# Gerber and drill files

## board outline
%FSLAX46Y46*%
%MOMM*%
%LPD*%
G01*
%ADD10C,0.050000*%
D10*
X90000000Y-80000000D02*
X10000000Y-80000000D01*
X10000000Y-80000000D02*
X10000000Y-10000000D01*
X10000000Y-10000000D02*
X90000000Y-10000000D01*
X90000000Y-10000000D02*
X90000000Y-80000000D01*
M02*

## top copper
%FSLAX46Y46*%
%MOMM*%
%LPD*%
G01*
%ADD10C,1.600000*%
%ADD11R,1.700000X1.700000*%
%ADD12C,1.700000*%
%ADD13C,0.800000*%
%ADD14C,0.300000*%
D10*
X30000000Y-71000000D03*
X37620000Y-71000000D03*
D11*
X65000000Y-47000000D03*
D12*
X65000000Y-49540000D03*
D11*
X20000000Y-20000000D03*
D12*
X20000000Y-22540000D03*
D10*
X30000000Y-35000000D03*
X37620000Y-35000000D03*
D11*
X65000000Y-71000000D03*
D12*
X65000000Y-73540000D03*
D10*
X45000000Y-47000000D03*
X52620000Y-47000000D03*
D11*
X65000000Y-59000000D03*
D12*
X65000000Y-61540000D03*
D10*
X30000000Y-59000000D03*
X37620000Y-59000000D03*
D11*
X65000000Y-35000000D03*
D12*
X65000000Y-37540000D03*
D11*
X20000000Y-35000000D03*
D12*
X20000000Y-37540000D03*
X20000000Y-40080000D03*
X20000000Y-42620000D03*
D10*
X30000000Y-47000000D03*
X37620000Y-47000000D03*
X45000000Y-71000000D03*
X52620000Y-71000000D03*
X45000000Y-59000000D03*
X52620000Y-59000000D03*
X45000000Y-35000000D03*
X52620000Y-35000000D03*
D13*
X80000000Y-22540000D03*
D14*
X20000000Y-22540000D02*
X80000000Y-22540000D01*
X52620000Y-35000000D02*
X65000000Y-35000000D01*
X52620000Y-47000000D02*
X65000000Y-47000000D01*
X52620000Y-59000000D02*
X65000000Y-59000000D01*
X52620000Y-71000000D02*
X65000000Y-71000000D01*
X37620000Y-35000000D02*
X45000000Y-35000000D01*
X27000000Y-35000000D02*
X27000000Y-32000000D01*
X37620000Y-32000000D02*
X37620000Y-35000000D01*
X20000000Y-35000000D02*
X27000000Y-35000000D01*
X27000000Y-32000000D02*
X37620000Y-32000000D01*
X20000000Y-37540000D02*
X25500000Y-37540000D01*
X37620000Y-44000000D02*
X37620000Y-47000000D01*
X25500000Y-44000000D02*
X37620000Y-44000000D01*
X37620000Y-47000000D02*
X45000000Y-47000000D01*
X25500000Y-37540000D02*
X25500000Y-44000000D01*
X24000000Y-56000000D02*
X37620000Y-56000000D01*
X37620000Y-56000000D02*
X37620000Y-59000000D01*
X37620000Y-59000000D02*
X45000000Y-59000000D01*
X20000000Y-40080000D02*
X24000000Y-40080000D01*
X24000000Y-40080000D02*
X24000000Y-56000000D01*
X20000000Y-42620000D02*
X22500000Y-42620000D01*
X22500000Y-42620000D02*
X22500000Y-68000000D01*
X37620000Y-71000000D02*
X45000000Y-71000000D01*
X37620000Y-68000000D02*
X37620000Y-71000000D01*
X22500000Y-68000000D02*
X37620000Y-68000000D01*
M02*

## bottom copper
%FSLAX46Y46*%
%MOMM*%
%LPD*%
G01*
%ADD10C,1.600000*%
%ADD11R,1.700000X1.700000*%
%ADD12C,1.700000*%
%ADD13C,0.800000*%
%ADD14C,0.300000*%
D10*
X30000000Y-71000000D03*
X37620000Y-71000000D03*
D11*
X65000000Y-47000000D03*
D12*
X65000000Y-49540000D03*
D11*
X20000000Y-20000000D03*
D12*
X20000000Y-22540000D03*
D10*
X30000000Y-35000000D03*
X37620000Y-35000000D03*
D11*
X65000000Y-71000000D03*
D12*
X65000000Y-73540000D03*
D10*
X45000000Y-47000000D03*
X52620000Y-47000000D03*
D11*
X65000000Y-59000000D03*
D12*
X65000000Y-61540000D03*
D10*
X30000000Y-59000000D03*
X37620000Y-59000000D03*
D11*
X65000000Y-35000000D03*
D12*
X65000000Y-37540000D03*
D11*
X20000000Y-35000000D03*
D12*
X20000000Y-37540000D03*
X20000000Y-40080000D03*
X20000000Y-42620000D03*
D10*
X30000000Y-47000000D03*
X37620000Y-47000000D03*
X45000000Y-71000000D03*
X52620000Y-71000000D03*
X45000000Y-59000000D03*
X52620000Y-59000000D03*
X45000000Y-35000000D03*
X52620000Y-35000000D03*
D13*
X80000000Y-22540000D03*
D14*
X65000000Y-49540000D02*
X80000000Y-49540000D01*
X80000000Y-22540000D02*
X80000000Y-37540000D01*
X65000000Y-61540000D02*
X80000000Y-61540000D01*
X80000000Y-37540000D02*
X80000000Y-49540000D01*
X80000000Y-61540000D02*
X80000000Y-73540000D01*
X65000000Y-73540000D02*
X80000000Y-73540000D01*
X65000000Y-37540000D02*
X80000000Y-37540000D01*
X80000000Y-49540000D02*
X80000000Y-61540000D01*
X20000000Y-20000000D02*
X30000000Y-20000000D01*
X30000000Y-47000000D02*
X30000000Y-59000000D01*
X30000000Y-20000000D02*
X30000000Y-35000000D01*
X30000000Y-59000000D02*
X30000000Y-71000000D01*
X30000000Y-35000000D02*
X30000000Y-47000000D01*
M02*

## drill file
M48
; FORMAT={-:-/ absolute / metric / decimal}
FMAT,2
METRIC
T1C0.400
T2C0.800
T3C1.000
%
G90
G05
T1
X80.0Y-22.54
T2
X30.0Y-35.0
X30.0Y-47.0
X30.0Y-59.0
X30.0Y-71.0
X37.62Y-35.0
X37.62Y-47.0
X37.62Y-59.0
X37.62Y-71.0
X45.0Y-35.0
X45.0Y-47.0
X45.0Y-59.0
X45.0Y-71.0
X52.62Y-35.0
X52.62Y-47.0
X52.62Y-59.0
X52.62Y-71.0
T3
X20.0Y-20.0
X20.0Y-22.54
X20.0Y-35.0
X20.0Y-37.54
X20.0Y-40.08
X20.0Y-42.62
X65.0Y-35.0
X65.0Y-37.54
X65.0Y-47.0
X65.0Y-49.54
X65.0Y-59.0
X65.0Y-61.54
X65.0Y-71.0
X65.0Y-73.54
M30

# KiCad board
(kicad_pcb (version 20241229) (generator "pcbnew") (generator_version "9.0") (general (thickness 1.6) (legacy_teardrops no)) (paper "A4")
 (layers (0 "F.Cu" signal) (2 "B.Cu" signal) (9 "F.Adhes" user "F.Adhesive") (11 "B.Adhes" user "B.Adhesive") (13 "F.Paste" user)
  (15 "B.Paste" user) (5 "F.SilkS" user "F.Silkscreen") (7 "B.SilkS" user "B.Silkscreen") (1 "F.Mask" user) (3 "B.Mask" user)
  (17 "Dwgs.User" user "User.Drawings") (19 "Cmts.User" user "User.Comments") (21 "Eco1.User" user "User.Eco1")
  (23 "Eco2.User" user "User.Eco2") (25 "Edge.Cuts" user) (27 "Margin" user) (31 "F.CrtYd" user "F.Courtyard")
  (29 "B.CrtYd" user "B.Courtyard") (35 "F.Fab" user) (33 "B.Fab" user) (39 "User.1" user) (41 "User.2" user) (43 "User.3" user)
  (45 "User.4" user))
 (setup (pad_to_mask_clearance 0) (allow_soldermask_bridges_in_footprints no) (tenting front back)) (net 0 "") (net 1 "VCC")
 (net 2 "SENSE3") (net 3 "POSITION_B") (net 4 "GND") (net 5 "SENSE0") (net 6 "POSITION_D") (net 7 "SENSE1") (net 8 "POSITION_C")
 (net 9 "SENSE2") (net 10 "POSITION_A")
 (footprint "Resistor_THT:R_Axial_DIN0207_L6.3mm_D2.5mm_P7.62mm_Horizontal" (layer "F.Cu") (at 30 71)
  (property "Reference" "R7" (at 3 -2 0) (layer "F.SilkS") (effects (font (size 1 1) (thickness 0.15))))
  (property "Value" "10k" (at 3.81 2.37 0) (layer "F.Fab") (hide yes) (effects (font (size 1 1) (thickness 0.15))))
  (pad "1" thru_hole circle (at 0 0) (size 1.6 1.6) (drill 0.8) (layers "*.Cu" "*.Mask") (remove_unused_layers no) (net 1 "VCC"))
  (pad "2" thru_hole circle (at 7.62 0) (size 1.6 1.6) (drill 0.8) (layers "*.Cu" "*.Mask") (remove_unused_layers no) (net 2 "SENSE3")))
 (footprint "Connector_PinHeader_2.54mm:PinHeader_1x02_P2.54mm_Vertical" (layer "F.Cu") (at 65 47)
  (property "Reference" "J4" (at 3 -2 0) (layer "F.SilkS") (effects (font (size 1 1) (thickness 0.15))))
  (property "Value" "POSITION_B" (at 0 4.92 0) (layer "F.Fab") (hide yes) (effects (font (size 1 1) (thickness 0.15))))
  (pad "1" thru_hole rect (at 0 0) (size 1.7 1.7) (drill 1) (layers "*.Cu" "*.Mask") (remove_unused_layers no) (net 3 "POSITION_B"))
  (pad "2" thru_hole circle (at 0 2.54) (size 1.7 1.7) (drill 1) (layers "*.Cu" "*.Mask") (remove_unused_layers no) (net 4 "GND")))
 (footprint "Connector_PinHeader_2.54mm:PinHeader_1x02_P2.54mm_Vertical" (layer "F.Cu") (at 20 20)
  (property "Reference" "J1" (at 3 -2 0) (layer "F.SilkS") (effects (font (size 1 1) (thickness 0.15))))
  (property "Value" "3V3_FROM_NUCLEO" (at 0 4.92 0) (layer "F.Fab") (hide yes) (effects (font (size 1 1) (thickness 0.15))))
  (pad "1" thru_hole rect (at 0 0) (size 1.7 1.7) (drill 1) (layers "*.Cu" "*.Mask") (remove_unused_layers no) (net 1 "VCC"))
  (pad "2" thru_hole circle (at 0 2.54) (size 1.7 1.7) (drill 1) (layers "*.Cu" "*.Mask") (remove_unused_layers no) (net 4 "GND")))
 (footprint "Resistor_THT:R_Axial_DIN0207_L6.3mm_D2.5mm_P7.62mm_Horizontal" (layer "F.Cu") (at 30 35)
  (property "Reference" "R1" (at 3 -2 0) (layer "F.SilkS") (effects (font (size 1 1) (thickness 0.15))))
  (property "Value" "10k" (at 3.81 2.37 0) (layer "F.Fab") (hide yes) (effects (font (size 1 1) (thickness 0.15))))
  (pad "1" thru_hole circle (at 0 0) (size 1.6 1.6) (drill 0.8) (layers "*.Cu" "*.Mask") (remove_unused_layers no) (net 1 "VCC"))
  (pad "2" thru_hole circle (at 7.62 0) (size 1.6 1.6) (drill 0.8) (layers "*.Cu" "*.Mask") (remove_unused_layers no) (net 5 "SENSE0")))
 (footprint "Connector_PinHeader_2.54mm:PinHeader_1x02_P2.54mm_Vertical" (layer "F.Cu") (at 65 71)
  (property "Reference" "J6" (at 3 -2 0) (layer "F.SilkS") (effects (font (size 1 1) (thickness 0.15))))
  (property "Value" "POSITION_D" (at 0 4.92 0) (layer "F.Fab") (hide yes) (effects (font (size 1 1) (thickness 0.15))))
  (pad "1" thru_hole rect (at 0 0) (size 1.7 1.7) (drill 1) (layers "*.Cu" "*.Mask") (remove_unused_layers no) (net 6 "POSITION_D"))
  (pad "2" thru_hole circle (at 0 2.54) (size 1.7 1.7) (drill 1) (layers "*.Cu" "*.Mask") (remove_unused_layers no) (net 4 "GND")))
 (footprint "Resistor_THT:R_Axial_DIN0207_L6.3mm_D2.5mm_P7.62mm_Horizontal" (layer "F.Cu") (at 45 47)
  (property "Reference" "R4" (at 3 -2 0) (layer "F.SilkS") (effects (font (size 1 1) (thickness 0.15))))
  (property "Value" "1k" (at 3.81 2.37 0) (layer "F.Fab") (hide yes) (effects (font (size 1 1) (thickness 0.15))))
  (pad "1" thru_hole circle (at 0 0) (size 1.6 1.6) (drill 0.8) (layers "*.Cu" "*.Mask") (remove_unused_layers no) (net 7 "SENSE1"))
  (pad "2" thru_hole circle (at 7.62 0) (size 1.6 1.6) (drill 0.8) (layers "*.Cu" "*.Mask") (remove_unused_layers no) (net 3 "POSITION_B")))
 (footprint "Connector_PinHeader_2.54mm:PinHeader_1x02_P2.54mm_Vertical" (layer "F.Cu") (at 65 59)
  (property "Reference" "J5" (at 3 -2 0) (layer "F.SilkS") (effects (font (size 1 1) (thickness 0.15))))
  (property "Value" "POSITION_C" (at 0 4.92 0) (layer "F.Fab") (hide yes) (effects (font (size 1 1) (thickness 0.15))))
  (pad "1" thru_hole rect (at 0 0) (size 1.7 1.7) (drill 1) (layers "*.Cu" "*.Mask") (remove_unused_layers no) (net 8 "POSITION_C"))
  (pad "2" thru_hole circle (at 0 2.54) (size 1.7 1.7) (drill 1) (layers "*.Cu" "*.Mask") (remove_unused_layers no) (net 4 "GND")))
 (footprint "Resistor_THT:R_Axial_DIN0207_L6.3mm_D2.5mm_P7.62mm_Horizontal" (layer "F.Cu") (at 30 59)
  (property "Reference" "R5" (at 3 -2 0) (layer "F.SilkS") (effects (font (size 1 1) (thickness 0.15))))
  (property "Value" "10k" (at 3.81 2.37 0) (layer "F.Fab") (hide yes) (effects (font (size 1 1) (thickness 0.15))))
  (pad "1" thru_hole circle (at 0 0) (size 1.6 1.6) (drill 0.8) (layers "*.Cu" "*.Mask") (remove_unused_layers no) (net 1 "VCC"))
  (pad "2" thru_hole circle (at 7.62 0) (size 1.6 1.6) (drill 0.8) (layers "*.Cu" "*.Mask") (remove_unused_layers no) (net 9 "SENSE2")))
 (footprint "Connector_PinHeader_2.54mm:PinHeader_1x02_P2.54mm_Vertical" (layer "F.Cu") (at 65 35)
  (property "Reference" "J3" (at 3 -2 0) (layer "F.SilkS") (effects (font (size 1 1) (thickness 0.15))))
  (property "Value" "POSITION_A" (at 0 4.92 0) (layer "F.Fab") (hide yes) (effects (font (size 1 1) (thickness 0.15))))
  (pad "1" thru_hole rect (at 0 0) (size 1.7 1.7) (drill 1) (layers "*.Cu" "*.Mask") (remove_unused_layers no) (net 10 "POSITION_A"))
  (pad "2" thru_hole circle (at 0 2.54) (size 1.7 1.7) (drill 1) (layers "*.Cu" "*.Mask") (remove_unused_layers no) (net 4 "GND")))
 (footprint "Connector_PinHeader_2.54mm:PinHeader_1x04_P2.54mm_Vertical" (layer "F.Cu") (at 20 35)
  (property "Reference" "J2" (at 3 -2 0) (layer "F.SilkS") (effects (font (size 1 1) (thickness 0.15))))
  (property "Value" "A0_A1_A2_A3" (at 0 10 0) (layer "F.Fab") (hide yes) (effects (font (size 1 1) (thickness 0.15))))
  (pad "1" thru_hole rect (at 0 0) (size 1.7 1.7) (drill 1) (layers "*.Cu" "*.Mask") (remove_unused_layers no) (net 5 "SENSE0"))
  (pad "2" thru_hole circle (at 0 2.54) (size 1.7 1.7) (drill 1) (layers "*.Cu" "*.Mask") (remove_unused_layers no) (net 7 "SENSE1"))
  (pad "3" thru_hole circle (at 0 5.08) (size 1.7 1.7) (drill 1) (layers "*.Cu" "*.Mask") (remove_unused_layers no) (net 9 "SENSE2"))
  (pad "4" thru_hole circle (at 0 7.62) (size 1.7 1.7) (drill 1) (layers "*.Cu" "*.Mask") (remove_unused_layers no) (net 2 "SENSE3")))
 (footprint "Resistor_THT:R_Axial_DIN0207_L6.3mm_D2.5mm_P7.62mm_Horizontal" (layer "F.Cu") (at 30 47)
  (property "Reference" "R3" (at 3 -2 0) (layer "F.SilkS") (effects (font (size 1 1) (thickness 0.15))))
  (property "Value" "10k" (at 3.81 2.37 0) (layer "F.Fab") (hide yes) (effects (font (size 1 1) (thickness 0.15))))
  (pad "1" thru_hole circle (at 0 0) (size 1.6 1.6) (drill 0.8) (layers "*.Cu" "*.Mask") (remove_unused_layers no) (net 1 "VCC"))
  (pad "2" thru_hole circle (at 7.62 0) (size 1.6 1.6) (drill 0.8) (layers "*.Cu" "*.Mask") (remove_unused_layers no) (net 7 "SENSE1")))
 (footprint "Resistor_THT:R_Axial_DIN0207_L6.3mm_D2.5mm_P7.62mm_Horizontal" (layer "F.Cu") (at 45 71)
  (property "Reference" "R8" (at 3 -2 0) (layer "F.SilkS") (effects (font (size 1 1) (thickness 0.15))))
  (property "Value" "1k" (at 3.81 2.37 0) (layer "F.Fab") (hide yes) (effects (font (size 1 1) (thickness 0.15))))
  (pad "1" thru_hole circle (at 0 0) (size 1.6 1.6) (drill 0.8) (layers "*.Cu" "*.Mask") (remove_unused_layers no) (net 2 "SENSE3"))
  (pad "2" thru_hole circle (at 7.62 0) (size 1.6 1.6) (drill 0.8) (layers "*.Cu" "*.Mask") (remove_unused_layers no) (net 6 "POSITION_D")))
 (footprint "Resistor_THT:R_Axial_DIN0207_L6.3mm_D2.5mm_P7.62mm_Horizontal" (layer "F.Cu") (at 45 59)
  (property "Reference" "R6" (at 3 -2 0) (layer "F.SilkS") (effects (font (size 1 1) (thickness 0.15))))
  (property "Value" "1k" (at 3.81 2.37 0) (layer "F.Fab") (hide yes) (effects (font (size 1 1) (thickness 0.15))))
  (pad "1" thru_hole circle (at 0 0) (size 1.6 1.6) (drill 0.8) (layers "*.Cu" "*.Mask") (remove_unused_layers no) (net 9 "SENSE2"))
  (pad "2" thru_hole circle (at 7.62 0) (size 1.6 1.6) (drill 0.8) (layers "*.Cu" "*.Mask") (remove_unused_layers no) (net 8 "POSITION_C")))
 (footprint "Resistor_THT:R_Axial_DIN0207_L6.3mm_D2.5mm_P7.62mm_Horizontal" (layer "F.Cu") (at 45 35)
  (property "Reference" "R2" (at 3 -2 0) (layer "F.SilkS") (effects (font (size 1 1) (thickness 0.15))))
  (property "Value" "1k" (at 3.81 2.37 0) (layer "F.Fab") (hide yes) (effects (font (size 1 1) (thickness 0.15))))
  (pad "1" thru_hole circle (at 0 0) (size 1.6 1.6) (drill 0.8) (layers "*.Cu" "*.Mask") (remove_unused_layers no) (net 5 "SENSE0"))
  (pad "2" thru_hole circle (at 7.62 0) (size 1.6 1.6) (drill 0.8) (layers "*.Cu" "*.Mask") (remove_unused_layers no) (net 10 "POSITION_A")))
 (gr_line (start 90 80) (end 10 80) (stroke (width 0.05) (type default)) (layer "Edge.Cuts"))
 (gr_line (start 10 80) (end 10 10) (stroke (width 0.05) (type default)) (layer "Edge.Cuts"))
 (gr_line (start 10 10) (end 90 10) (stroke (width 0.05) (type default)) (layer "Edge.Cuts"))
 (gr_line (start 90 10) (end 90 80) (stroke (width 0.05) (type default)) (layer "Edge.Cuts"))
 (segment (start 20 22.54) (end 80 22.54) (width 0.3) (layer "F.Cu") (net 4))
 (via (at 80 22.54) (size 0.8) (drill 0.4) (layers "F.Cu" "B.Cu") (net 4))
 (segment (start 65 49.54) (end 80 49.54) (width 0.3) (layer "B.Cu") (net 4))
 (segment (start 80 22.54) (end 80 37.54) (width 0.3) (layer "B.Cu") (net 4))
 (segment (start 65 61.54) (end 80 61.54) (width 0.3) (layer "B.Cu") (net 4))
 (segment (start 80 37.54) (end 80 49.54) (width 0.3) (layer "B.Cu") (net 4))
 (segment (start 80 61.54) (end 80 73.54) (width 0.3) (layer "B.Cu") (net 4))
 (segment (start 65 73.54) (end 80 73.54) (width 0.3) (layer "B.Cu") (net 4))
 (segment (start 65 37.54) (end 80 37.54) (width 0.3) (layer "B.Cu") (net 4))
 (segment (start 80 49.54) (end 80 61.54) (width 0.3) (layer "B.Cu") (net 4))
 (segment (start 52.62 35) (end 65 35) (width 0.3) (layer "F.Cu") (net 10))
 (segment (start 52.62 47) (end 65 47) (width 0.3) (layer "F.Cu") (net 3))
 (segment (start 52.62 59) (end 65 59) (width 0.3) (layer "F.Cu") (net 8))
 (segment (start 52.62 71) (end 65 71) (width 0.3) (layer "F.Cu") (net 6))
 (segment (start 37.62 35) (end 45 35) (width 0.3) (layer "F.Cu") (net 5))
 (segment (start 27 35) (end 27 32) (width 0.3) (layer "F.Cu") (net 5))
 (segment (start 37.62 32) (end 37.62 35) (width 0.3) (layer "F.Cu") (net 5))
 (segment (start 20 35) (end 27 35) (width 0.3) (layer "F.Cu") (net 5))
 (segment (start 27 32) (end 37.62 32) (width 0.3) (layer "F.Cu") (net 5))
 (segment (start 20 37.54) (end 25.5 37.54) (width 0.3) (layer "F.Cu") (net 7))
 (segment (start 37.62 44) (end 37.62 47) (width 0.3) (layer "F.Cu") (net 7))
 (segment (start 25.5 44) (end 37.62 44) (width 0.3) (layer "F.Cu") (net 7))
 (segment (start 37.62 47) (end 45 47) (width 0.3) (layer "F.Cu") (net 7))
 (segment (start 25.5 37.54) (end 25.5 44) (width 0.3) (layer "F.Cu") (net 7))
 (segment (start 24 56) (end 37.62 56) (width 0.3) (layer "F.Cu") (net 9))
 (segment (start 37.62 56) (end 37.62 59) (width 0.3) (layer "F.Cu") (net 9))
 (segment (start 37.62 59) (end 45 59) (width 0.3) (layer "F.Cu") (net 9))
 (segment (start 20 40.08) (end 24 40.08) (width 0.3) (layer "F.Cu") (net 9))
 (segment (start 24 40.08) (end 24 56) (width 0.3) (layer "F.Cu") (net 9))
 (segment (start 20 42.62) (end 22.5 42.62) (width 0.3) (layer "F.Cu") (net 2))
 (segment (start 22.5 42.62) (end 22.5 68) (width 0.3) (layer "F.Cu") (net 2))
 (segment (start 37.62 71) (end 45 71) (width 0.3) (layer "F.Cu") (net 2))
 (segment (start 37.62 68) (end 37.62 71) (width 0.3) (layer "F.Cu") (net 2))
 (segment (start 22.5 68) (end 37.62 68) (width 0.3) (layer "F.Cu") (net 2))
 (segment (start 20 20) (end 30 20) (width 0.3) (layer "B.Cu") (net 1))
 (segment (start 30 47) (end 30 59) (width 0.3) (layer "B.Cu") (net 1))
 (segment (start 30 20) (end 30 35) (width 0.3) (layer "B.Cu") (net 1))
 (segment (start 30 59) (end 30 71) (width 0.3) (layer "B.Cu") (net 1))
 (segment (start 30 35) (end 30 47) (width 0.3) (layer "B.Cu") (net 1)))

